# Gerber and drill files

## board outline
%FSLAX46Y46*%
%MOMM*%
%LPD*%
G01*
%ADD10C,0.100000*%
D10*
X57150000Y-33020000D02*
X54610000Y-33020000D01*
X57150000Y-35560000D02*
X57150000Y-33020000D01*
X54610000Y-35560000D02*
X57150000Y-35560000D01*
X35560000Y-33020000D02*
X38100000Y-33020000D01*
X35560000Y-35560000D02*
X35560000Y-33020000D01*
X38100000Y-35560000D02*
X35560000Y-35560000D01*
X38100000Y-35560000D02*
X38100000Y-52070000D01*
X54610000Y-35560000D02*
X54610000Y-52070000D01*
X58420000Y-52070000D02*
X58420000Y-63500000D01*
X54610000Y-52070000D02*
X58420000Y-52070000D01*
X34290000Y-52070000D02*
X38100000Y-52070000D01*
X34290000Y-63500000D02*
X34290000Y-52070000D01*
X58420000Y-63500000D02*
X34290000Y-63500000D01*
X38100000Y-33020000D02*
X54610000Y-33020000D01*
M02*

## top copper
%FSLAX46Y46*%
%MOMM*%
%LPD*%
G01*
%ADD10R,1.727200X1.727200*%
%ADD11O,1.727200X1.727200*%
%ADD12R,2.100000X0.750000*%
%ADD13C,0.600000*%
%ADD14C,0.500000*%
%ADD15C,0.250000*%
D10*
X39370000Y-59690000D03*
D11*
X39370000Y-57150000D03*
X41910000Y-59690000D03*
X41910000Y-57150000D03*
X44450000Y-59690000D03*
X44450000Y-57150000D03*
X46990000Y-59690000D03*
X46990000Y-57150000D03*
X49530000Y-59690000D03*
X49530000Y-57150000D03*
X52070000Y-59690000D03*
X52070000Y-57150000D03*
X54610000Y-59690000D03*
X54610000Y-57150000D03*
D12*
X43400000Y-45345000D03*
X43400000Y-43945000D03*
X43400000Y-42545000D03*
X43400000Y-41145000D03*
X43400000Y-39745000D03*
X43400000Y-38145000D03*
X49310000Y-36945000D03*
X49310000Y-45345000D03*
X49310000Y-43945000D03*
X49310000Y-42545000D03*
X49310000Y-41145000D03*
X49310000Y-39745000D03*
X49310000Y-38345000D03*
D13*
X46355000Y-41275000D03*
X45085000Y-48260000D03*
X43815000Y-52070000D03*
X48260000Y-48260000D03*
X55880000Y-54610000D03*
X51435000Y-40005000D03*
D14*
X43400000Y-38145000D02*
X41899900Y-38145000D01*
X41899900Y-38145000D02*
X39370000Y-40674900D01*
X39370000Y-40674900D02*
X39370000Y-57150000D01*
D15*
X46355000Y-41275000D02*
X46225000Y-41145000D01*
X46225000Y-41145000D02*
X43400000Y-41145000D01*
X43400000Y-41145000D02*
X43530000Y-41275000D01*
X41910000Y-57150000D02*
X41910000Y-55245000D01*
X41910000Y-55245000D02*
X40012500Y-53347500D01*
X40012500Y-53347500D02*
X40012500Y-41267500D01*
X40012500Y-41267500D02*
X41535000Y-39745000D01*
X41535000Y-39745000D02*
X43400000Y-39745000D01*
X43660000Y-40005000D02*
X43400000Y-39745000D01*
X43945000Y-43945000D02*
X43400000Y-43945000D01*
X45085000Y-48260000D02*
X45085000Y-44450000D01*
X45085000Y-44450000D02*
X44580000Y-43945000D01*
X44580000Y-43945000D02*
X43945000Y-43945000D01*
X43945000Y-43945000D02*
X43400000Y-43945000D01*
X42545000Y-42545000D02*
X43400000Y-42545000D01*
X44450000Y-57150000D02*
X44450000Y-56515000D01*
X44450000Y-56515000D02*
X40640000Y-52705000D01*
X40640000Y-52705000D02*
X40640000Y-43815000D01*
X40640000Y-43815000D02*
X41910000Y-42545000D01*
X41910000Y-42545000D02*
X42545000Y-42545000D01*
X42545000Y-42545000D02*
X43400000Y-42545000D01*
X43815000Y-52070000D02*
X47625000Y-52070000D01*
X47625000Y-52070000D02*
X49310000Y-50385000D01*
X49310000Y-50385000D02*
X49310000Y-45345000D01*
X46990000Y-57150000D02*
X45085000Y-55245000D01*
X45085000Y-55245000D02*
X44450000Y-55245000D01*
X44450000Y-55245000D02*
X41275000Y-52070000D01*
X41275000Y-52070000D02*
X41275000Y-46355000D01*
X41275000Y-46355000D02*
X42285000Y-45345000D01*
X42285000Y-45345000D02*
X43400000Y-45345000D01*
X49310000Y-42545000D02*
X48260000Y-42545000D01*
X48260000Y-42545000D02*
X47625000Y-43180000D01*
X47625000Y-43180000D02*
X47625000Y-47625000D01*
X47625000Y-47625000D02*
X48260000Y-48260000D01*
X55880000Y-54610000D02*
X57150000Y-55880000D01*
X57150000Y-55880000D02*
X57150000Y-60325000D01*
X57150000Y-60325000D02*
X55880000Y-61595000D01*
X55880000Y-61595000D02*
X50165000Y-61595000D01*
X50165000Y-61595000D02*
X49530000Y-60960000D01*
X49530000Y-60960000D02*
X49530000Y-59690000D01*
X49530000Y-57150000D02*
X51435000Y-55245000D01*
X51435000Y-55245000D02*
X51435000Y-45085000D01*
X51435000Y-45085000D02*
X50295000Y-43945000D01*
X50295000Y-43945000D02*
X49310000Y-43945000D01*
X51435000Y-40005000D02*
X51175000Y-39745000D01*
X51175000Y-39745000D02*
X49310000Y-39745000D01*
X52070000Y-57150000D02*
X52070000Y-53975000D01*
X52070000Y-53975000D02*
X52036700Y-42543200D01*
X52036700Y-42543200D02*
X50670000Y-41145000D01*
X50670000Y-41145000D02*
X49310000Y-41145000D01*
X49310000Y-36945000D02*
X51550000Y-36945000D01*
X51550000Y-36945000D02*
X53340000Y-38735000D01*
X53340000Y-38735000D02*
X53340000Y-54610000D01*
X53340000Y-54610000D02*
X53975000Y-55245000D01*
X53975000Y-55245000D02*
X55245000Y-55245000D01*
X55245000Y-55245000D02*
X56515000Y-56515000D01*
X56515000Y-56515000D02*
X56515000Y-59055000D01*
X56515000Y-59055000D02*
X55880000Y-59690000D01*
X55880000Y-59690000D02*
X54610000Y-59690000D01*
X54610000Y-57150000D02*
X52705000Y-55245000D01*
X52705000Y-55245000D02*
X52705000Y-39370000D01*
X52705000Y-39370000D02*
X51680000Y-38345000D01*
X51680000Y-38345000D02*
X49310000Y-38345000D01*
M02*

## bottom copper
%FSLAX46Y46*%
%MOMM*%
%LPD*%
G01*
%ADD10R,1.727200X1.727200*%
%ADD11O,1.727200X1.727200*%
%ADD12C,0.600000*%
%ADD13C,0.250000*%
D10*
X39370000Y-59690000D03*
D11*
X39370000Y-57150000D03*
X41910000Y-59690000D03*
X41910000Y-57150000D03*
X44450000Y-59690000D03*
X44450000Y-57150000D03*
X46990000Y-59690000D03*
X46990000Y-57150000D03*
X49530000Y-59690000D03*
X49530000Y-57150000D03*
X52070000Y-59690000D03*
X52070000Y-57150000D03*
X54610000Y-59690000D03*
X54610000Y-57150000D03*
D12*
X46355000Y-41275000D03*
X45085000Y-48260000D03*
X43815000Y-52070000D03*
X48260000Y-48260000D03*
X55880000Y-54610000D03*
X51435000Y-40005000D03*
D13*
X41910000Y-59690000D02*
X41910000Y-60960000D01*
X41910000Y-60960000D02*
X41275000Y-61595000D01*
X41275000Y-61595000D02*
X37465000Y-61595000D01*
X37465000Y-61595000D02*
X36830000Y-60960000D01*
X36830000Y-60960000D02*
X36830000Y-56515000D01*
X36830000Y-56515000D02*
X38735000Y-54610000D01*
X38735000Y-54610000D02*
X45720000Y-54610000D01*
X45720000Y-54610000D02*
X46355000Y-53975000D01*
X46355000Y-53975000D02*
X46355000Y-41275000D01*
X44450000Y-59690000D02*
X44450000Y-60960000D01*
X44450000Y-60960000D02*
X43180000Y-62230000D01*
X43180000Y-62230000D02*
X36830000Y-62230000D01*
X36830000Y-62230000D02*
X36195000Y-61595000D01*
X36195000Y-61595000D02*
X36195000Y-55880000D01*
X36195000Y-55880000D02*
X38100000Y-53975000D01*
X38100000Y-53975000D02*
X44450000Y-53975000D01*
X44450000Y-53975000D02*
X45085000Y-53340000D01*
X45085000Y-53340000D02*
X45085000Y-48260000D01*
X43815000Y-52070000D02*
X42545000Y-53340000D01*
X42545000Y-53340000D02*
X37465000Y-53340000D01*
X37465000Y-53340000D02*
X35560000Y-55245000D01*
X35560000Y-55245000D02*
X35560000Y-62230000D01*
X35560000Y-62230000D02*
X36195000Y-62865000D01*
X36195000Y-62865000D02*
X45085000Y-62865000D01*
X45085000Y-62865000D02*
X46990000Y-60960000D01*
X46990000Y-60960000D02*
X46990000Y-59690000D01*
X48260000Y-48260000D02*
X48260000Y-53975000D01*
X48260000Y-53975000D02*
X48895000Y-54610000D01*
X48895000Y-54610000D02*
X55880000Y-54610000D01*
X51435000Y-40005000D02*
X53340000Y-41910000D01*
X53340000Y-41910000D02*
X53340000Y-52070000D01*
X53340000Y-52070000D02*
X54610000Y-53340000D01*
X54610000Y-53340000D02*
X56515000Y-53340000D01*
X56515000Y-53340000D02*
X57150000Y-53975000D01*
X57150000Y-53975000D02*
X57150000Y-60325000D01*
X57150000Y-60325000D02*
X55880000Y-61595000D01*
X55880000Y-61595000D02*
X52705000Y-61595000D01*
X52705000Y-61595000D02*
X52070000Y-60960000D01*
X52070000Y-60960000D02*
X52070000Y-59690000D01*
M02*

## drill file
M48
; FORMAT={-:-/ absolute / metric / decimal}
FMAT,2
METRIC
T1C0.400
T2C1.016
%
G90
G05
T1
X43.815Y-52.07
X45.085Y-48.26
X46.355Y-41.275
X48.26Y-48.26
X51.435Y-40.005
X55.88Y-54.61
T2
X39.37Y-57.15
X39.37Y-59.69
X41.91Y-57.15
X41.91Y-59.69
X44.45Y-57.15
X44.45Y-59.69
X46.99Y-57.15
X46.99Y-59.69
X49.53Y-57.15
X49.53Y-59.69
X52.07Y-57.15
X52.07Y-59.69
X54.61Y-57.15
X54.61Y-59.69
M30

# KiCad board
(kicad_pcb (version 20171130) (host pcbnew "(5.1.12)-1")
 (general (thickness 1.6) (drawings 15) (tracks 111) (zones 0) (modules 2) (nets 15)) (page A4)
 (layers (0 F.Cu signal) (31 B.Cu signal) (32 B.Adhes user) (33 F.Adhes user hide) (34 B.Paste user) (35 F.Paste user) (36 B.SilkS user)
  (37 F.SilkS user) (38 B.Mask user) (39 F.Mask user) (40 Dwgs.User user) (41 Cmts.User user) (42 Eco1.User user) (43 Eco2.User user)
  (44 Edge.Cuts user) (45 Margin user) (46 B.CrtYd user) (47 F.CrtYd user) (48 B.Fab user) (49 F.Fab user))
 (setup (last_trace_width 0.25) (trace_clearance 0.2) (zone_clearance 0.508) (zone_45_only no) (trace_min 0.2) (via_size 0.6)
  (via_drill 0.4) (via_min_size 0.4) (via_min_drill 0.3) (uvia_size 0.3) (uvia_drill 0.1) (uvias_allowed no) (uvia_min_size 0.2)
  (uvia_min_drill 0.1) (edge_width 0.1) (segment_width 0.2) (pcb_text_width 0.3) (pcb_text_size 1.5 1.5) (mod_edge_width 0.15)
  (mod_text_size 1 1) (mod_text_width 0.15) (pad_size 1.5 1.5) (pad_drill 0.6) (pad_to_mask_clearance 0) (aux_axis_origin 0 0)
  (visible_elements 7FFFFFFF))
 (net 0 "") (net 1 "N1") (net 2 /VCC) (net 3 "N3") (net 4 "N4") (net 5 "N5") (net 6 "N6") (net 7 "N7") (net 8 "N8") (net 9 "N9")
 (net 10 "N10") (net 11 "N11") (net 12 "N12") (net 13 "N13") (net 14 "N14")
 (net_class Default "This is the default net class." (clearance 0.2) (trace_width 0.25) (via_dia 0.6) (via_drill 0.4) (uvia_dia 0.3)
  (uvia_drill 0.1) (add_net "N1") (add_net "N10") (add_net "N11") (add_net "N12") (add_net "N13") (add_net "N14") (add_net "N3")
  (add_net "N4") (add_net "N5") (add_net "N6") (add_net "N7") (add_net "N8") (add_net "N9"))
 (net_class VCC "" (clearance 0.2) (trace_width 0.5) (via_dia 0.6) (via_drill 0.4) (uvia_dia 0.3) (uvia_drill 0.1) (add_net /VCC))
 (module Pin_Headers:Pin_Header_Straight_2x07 (layer F.Cu) (at 39.37 59.69 90)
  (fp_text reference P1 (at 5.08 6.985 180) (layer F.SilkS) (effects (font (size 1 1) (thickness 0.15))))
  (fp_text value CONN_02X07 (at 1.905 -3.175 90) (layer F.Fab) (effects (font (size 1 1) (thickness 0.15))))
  (pad 1 thru_hole rect (at 0 0 90) (size 1.7272 1.7272) (drill 1.016) (layers *.Cu *.Mask F.SilkS) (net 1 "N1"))
  (pad 2 thru_hole oval (at 2.54 0 90) (size 1.7272 1.7272) (drill 1.016) (layers *.Cu *.Mask F.SilkS) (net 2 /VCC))
  (pad 3 thru_hole oval (at 0 2.54 90) (size 1.7272 1.7272) (drill 1.016) (layers *.Cu *.Mask F.SilkS) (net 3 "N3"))
  (pad 4 thru_hole oval (at 2.54 2.54 90) (size 1.7272 1.7272) (drill 1.016) (layers *.Cu *.Mask F.SilkS) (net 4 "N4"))
  (pad 5 thru_hole oval (at 0 5.08 90) (size 1.7272 1.7272) (drill 1.016) (layers *.Cu *.Mask F.SilkS) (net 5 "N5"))
  (pad 6 thru_hole oval (at 2.54 5.08 90) (size 1.7272 1.7272) (drill 1.016) (layers *.Cu *.Mask F.SilkS) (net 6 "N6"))
  (pad 7 thru_hole oval (at 0 7.62 90) (size 1.7272 1.7272) (drill 1.016) (layers *.Cu *.Mask F.SilkS) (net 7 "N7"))
  (pad 8 thru_hole oval (at 2.54 7.62 90) (size 1.7272 1.7272) (drill 1.016) (layers *.Cu *.Mask F.SilkS) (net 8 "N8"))
  (pad 9 thru_hole oval (at 0 10.16 90) (size 1.7272 1.7272) (drill 1.016) (layers *.Cu *.Mask F.SilkS) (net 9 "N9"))
  (pad 10 thru_hole oval (at 2.54 10.16 90) (size 1.7272 1.7272) (drill 1.016) (layers *.Cu *.Mask F.SilkS) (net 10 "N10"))
  (pad 11 thru_hole oval (at 0 12.7 90) (size 1.7272 1.7272) (drill 1.016) (layers *.Cu *.Mask F.SilkS) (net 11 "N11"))
  (pad 12 thru_hole oval (at 2.54 12.7 90) (size 1.7272 1.7272) (drill 1.016) (layers *.Cu *.Mask F.SilkS) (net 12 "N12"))
  (pad 13 thru_hole oval (at 0 15.24 90) (size 1.7272 1.7272) (drill 1.016) (layers *.Cu *.Mask F.SilkS) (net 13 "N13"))
  (pad 14 thru_hole oval (at 2.54 15.24 90) (size 1.7272 1.7272) (drill 1.016) (layers *.Cu *.Mask F.SilkS) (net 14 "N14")))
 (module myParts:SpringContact (layer F.Cu) (at 44.45 45.72)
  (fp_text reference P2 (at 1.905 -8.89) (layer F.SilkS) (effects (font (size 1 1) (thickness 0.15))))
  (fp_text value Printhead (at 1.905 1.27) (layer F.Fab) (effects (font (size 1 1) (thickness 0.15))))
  (pad 5 smd rect (at -1.05 -0.375) (size 2.1 0.75) (layers F.Cu F.Paste F.Mask) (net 8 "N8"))
  (pad 4 smd rect (at -1.05 -1.775) (size 2.1 0.75) (layers F.Cu F.Paste F.Mask) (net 5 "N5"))
  (pad 3 smd rect (at -1.05 -3.175) (size 2.1 0.75) (layers F.Cu F.Paste F.Mask) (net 6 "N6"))
  (pad 2 smd rect (at -1.05 -4.575) (size 2.1 0.75) (layers F.Cu F.Paste F.Mask) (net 3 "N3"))
  (pad 1 smd rect (at -1.05 -5.975) (size 2.1 0.75) (layers F.Cu F.Paste F.Mask) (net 4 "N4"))
  (pad 13 smd rect (at -1.05 -7.575) (size 2.1 0.75) (layers F.Cu F.Paste F.Mask) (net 2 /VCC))
  (pad 12 smd rect (at 4.86 -8.775) (size 2.1 0.75) (layers F.Cu F.Paste F.Mask) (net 13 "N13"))
  (pad 6 smd rect (at 4.86 -0.375) (size 2.1 0.75) (layers F.Cu F.Paste F.Mask) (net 7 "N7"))
  (pad 7 smd rect (at 4.86 -1.775) (size 2.1 0.75) (layers F.Cu F.Paste F.Mask) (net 10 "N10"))
  (pad 8 smd rect (at 4.86 -3.175) (size 2.1 0.75) (layers F.Cu F.Paste F.Mask) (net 9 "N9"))
  (pad 9 smd rect (at 4.86 -4.575) (size 2.1 0.75) (layers F.Cu F.Paste F.Mask) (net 12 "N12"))
  (pad 10 smd rect (at 4.86 -5.975) (size 2.1 0.75) (layers F.Cu F.Paste F.Mask) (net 11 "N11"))
  (pad 11 smd rect (at 4.86 -7.375) (size 2.1 0.75) (layers F.Cu F.Paste F.Mask) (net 14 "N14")))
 (gr_line (start 57.15 33.02) (end 54.61 33.02) (angle 90) (layer Edge.Cuts) (width 0.1))
 (gr_line (start 57.15 35.56) (end 57.15 33.02) (angle 90) (layer Edge.Cuts) (width 0.1))
 (gr_line (start 54.61 35.56) (end 57.15 35.56) (angle 90) (layer Edge.Cuts) (width 0.1))
 (gr_line (start 35.56 33.02) (end 38.1 33.02) (angle 90) (layer Edge.Cuts) (width 0.1))
 (gr_line (start 35.56 35.56) (end 35.56 33.02) (angle 90) (layer Edge.Cuts) (width 0.1))
 (gr_line (start 38.1 35.56) (end 35.56 35.56) (angle 90) (layer Edge.Cuts) (width 0.1))
 (gr_line (start 38.1 35.56) (end 38.1 52.07) (angle 90) (layer Edge.Cuts) (width 0.1))
 (gr_line (start 54.61 35.56) (end 54.61 52.07) (angle 90) (layer Edge.Cuts) (width 0.1))
 (gr_line (start 58.42 52.07) (end 58.42 63.5) (angle 90) (layer Edge.Cuts) (width 0.1))
 (gr_line (start 54.61 52.07) (end 58.42 52.07) (angle 90) (layer Edge.Cuts) (width 0.1))
 (gr_line (start 34.29 52.07) (end 38.1 52.07) (angle 90) (layer Edge.Cuts) (width 0.1))
 (gr_line (start 34.29 63.5) (end 34.29 52.07) (angle 90) (layer Edge.Cuts) (width 0.1))
 (gr_line (start 58.42 63.5) (end 34.29 63.5) (angle 90) (layer Edge.Cuts) (width 0.1))
 (gr_line (start 38.1 33.02) (end 54.61 33.02) (angle 90) (layer Edge.Cuts) (width 0.1))
 (segment (start 43.4 38.145) (end 41.8999 38.145) (width 0.5) (layer F.Cu) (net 2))
 (segment (start 41.8999 38.145) (end 39.37 40.6749) (width 0.5) (layer F.Cu) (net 2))
 (segment (start 39.37 40.6749) (end 39.37 57.15) (width 0.5) (layer F.Cu) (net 2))
 (segment (start 46.355 41.275) (end 46.225 41.145) (width 0.25) (layer F.Cu) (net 3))
 (segment (start 46.225 41.145) (end 43.4 41.145) (width 0.25) (layer F.Cu) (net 3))
 (segment (start 41.91 59.69) (end 41.91 60.96) (width 0.25) (layer B.Cu) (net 3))
 (segment (start 41.91 60.96) (end 41.275 61.595) (width 0.25) (layer B.Cu) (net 3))
 (segment (start 41.275 61.595) (end 37.465 61.595) (width 0.25) (layer B.Cu) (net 3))
 (segment (start 37.465 61.595) (end 36.83 60.96) (width 0.25) (layer B.Cu) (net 3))
 (segment (start 36.83 60.96) (end 36.83 56.515) (width 0.25) (layer B.Cu) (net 3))
 (segment (start 36.83 56.515) (end 38.735 54.61) (width 0.25) (layer B.Cu) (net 3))
 (segment (start 38.735 54.61) (end 45.72 54.61) (width 0.25) (layer B.Cu) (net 3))
 (segment (start 45.72 54.61) (end 46.355 53.975) (width 0.25) (layer B.Cu) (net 3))
 (segment (start 46.355 53.975) (end 46.355 41.275) (width 0.25) (layer B.Cu) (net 3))
 (segment (start 43.4 41.145) (end 43.53 41.275) (width 0.25) (layer F.Cu) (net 3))
 (via (at 46.355 41.275) (size 0.6) (layers F.Cu B.Cu) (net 3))
 (segment (start 41.91 57.15) (end 41.91 55.245) (width 0.25) (layer F.Cu) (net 4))
 (segment (start 41.91 55.245) (end 40.0125 53.3475) (width 0.25) (layer F.Cu) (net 4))
 (segment (start 40.0125 53.3475) (end 40.0125 41.2675) (width 0.25) (layer F.Cu) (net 4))
 (segment (start 40.0125 41.2675) (end 41.535 39.745) (width 0.25) (layer F.Cu) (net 4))
 (segment (start 41.535 39.745) (end 43.4 39.745) (width 0.25) (layer F.Cu) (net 4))
 (segment (start 43.66 40.005) (end 43.4 39.745) (width 0.25) (layer F.Cu) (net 4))
 (segment (start 43.945 43.945) (end 43.4 43.945) (width 0.25) (layer F.Cu) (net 5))
 (segment (start 45.085 48.26) (end 45.085 44.45) (width 0.25) (layer F.Cu) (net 5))
 (segment (start 45.085 44.45) (end 44.58 43.945) (width 0.25) (layer F.Cu) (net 5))
 (segment (start 44.58 43.945) (end 43.945 43.945) (width 0.25) (layer F.Cu) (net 5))
 (segment (start 44.45 59.69) (end 44.45 60.96) (width 0.25) (layer B.Cu) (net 5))
 (segment (start 44.45 60.96) (end 43.18 62.23) (width 0.25) (layer B.Cu) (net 5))
 (segment (start 43.18 62.23) (end 36.83 62.23) (width 0.25) (layer B.Cu) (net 5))
 (segment (start 36.83 62.23) (end 36.195 61.595) (width 0.25) (layer B.Cu) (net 5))
 (segment (start 36.195 61.595) (end 36.195 55.88) (width 0.25) (layer B.Cu) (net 5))
 (segment (start 36.195 55.88) (end 38.1 53.975) (width 0.25) (layer B.Cu) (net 5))
 (segment (start 38.1 53.975) (end 44.45 53.975) (width 0.25) (layer B.Cu) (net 5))
 (segment (start 44.45 53.975) (end 45.085 53.34) (width 0.25) (layer B.Cu) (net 5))
 (segment (start 45.085 53.34) (end 45.085 48.26) (width 0.25) (layer B.Cu) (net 5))
 (segment (start 43.945 43.945) (end 43.4 43.945) (width 0.25) (layer F.Cu) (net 5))
 (via (at 45.085 48.26) (size 0.6) (layers F.Cu B.Cu) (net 5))
 (segment (start 42.545 42.545) (end 43.4 42.545) (width 0.25) (layer F.Cu) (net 6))
 (segment (start 44.45 57.15) (end 44.45 56.515) (width 0.25) (layer F.Cu) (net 6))
 (segment (start 44.45 56.515) (end 40.64 52.705) (width 0.25) (layer F.Cu) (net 6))
 (segment (start 40.64 52.705) (end 40.64 43.815) (width 0.25) (layer F.Cu) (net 6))
 (segment (start 40.64 43.815) (end 41.91 42.545) (width 0.25) (layer F.Cu) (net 6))
 (segment (start 41.91 42.545) (end 42.545 42.545) (width 0.25) (layer F.Cu) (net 6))
 (segment (start 42.545 42.545) (end 43.4 42.545) (width 0.25) (layer F.Cu) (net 6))
 (segment (start 43.815 52.07) (end 42.545 53.34) (width 0.25) (layer B.Cu) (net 7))
 (segment (start 42.545 53.34) (end 37.465 53.34) (width 0.25) (layer B.Cu) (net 7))
 (segment (start 37.465 53.34) (end 35.56 55.245) (width 0.25) (layer B.Cu) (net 7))
 (segment (start 35.56 55.245) (end 35.56 62.23) (width 0.25) (layer B.Cu) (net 7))
 (segment (start 35.56 62.23) (end 36.195 62.865) (width 0.25) (layer B.Cu) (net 7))
 (segment (start 36.195 62.865) (end 45.085 62.865) (width 0.25) (layer B.Cu) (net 7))
 (segment (start 45.085 62.865) (end 46.99 60.96) (width 0.25) (layer B.Cu) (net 7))
 (segment (start 46.99 60.96) (end 46.99 59.69) (width 0.25) (layer B.Cu) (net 7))
 (segment (start 43.815 52.07) (end 47.625 52.07) (width 0.25) (layer F.Cu) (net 7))
 (segment (start 47.625 52.07) (end 49.31 50.385) (width 0.25) (layer F.Cu) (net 7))
 (segment (start 49.31 50.385) (end 49.31 45.345) (width 0.25) (layer F.Cu) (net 7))
 (via (at 43.815 52.07) (size 0.6) (layers F.Cu B.Cu) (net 7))
 (segment (start 46.99 57.15) (end 45.085 55.245) (width 0.25) (layer F.Cu) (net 8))
 (segment (start 45.085 55.245) (end 44.45 55.245) (width 0.25) (layer F.Cu) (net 8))
 (segment (start 44.45 55.245) (end 41.275 52.07) (width 0.25) (layer F.Cu) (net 8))
 (segment (start 41.275 52.07) (end 41.275 46.355) (width 0.25) (layer F.Cu) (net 8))
 (segment (start 41.275 46.355) (end 42.285 45.345) (width 0.25) (layer F.Cu) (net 8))
 (segment (start 42.285 45.345) (end 43.4 45.345) (width 0.25) (layer F.Cu) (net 8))
 (segment (start 48.26 48.26) (end 48.26 53.975) (width 0.25) (layer B.Cu) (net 9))
 (segment (start 48.26 53.975) (end 48.895 54.61) (width 0.25) (layer B.Cu) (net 9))
 (segment (start 48.895 54.61) (end 55.88 54.61) (width 0.25) (layer B.Cu) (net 9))
 (segment (start 49.31 42.545) (end 48.26 42.545) (width 0.25) (layer F.Cu) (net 9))
 (segment (start 48.26 42.545) (end 47.625 43.18) (width 0.25) (layer F.Cu) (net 9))
 (segment (start 47.625 43.18) (end 47.625 47.625) (width 0.25) (layer F.Cu) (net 9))
 (segment (start 47.625 47.625) (end 48.26 48.26) (width 0.25) (layer F.Cu) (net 9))
 (segment (start 55.88 54.61) (end 57.15 55.88) (width 0.25) (layer F.Cu) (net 9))
 (segment (start 57.15 55.88) (end 57.15 60.325) (width 0.25) (layer F.Cu) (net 9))
 (segment (start 57.15 60.325) (end 55.88 61.595) (width 0.25) (layer F.Cu) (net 9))
 (segment (start 55.88 61.595) (end 50.165 61.595) (width 0.25) (layer F.Cu) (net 9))
 (segment (start 50.165 61.595) (end 49.53 60.96) (width 0.25) (layer F.Cu) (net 9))
 (segment (start 49.53 60.96) (end 49.53 59.69) (width 0.25) (layer F.Cu) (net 9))
 (via (at 48.26 48.26) (size 0.6) (layers F.Cu B.Cu) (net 9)) (via (at 55.88 54.61) (size 0.6) (layers F.Cu B.Cu) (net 9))
 (segment (start 49.53 57.15) (end 51.435 55.245) (width 0.25) (layer F.Cu) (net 10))
 (segment (start 51.435 55.245) (end 51.435 45.085) (width 0.25) (layer F.Cu) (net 10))
 (segment (start 51.435 45.085) (end 50.295 43.945) (width 0.25) (layer F.Cu) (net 10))
 (segment (start 50.295 43.945) (end 49.31 43.945) (width 0.25) (layer F.Cu) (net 10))
 (segment (start 51.435 40.005) (end 53.34 41.91) (width 0.25) (layer B.Cu) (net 11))
 (segment (start 53.34 41.91) (end 53.34 52.07) (width 0.25) (layer B.Cu) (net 11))
 (segment (start 53.34 52.07) (end 54.61 53.34) (width 0.25) (layer B.Cu) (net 11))
 (segment (start 54.61 53.34) (end 56.515 53.34) (width 0.25) (layer B.Cu) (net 11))
 (segment (start 56.515 53.34) (end 57.15 53.975) (width 0.25) (layer B.Cu) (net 11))
 (segment (start 57.15 53.975) (end 57.15 60.325) (width 0.25) (layer B.Cu) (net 11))
 (segment (start 57.15 60.325) (end 55.88 61.595) (width 0.25) (layer B.Cu) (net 11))
 (segment (start 55.88 61.595) (end 52.705 61.595) (width 0.25) (layer B.Cu) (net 11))
 (segment (start 52.705 61.595) (end 52.07 60.96) (width 0.25) (layer B.Cu) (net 11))
 (segment (start 52.07 60.96) (end 52.07 59.69) (width 0.25) (layer B.Cu) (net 11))
 (segment (start 51.435 40.005) (end 51.175 39.745) (width 0.25) (layer F.Cu) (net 11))
 (segment (start 51.175 39.745) (end 49.31 39.745) (width 0.25) (layer F.Cu) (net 11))
 (via (at 51.435 40.005) (size 0.6) (layers F.Cu B.Cu) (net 11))
 (segment (start 52.07 57.15) (end 52.07 53.975) (width 0.25) (layer F.Cu) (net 12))
 (segment (start 52.07 53.975) (end 52.0367 42.5432) (width 0.25) (layer F.Cu) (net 12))
 (segment (start 52.0367 42.5432) (end 50.67 41.145) (width 0.25) (layer F.Cu) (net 12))
 (segment (start 50.67 41.145) (end 49.31 41.145) (width 0.25) (layer F.Cu) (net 12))
 (segment (start 49.31 36.945) (end 51.55 36.945) (width 0.25) (layer F.Cu) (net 13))
 (segment (start 51.55 36.945) (end 53.34 38.735) (width 0.25) (layer F.Cu) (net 13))
 (segment (start 53.34 38.735) (end 53.34 54.61) (width 0.25) (layer F.Cu) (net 13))
 (segment (start 53.34 54.61) (end 53.975 55.245) (width 0.25) (layer F.Cu) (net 13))
 (segment (start 53.975 55.245) (end 55.245 55.245) (width 0.25) (layer F.Cu) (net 13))
 (segment (start 55.245 55.245) (end 56.515 56.515) (width 0.25) (layer F.Cu) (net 13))
 (segment (start 56.515 56.515) (end 56.515 59.055) (width 0.25) (layer F.Cu) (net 13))
 (segment (start 56.515 59.055) (end 55.88 59.69) (width 0.25) (layer F.Cu) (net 13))
 (segment (start 55.88 59.69) (end 54.61 59.69) (width 0.25) (layer F.Cu) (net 13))
 (segment (start 54.61 57.15) (end 52.705 55.245) (width 0.25) (layer F.Cu) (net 14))
 (segment (start 52.705 55.245) (end 52.705 39.37) (width 0.25) (layer F.Cu) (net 14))
 (segment (start 52.705 39.37) (end 51.68 38.345) (width 0.25) (layer F.Cu) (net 14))
 (segment (start 51.68 38.345) (end 49.31 38.345) (width 0.25) (layer F.Cu) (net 14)))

